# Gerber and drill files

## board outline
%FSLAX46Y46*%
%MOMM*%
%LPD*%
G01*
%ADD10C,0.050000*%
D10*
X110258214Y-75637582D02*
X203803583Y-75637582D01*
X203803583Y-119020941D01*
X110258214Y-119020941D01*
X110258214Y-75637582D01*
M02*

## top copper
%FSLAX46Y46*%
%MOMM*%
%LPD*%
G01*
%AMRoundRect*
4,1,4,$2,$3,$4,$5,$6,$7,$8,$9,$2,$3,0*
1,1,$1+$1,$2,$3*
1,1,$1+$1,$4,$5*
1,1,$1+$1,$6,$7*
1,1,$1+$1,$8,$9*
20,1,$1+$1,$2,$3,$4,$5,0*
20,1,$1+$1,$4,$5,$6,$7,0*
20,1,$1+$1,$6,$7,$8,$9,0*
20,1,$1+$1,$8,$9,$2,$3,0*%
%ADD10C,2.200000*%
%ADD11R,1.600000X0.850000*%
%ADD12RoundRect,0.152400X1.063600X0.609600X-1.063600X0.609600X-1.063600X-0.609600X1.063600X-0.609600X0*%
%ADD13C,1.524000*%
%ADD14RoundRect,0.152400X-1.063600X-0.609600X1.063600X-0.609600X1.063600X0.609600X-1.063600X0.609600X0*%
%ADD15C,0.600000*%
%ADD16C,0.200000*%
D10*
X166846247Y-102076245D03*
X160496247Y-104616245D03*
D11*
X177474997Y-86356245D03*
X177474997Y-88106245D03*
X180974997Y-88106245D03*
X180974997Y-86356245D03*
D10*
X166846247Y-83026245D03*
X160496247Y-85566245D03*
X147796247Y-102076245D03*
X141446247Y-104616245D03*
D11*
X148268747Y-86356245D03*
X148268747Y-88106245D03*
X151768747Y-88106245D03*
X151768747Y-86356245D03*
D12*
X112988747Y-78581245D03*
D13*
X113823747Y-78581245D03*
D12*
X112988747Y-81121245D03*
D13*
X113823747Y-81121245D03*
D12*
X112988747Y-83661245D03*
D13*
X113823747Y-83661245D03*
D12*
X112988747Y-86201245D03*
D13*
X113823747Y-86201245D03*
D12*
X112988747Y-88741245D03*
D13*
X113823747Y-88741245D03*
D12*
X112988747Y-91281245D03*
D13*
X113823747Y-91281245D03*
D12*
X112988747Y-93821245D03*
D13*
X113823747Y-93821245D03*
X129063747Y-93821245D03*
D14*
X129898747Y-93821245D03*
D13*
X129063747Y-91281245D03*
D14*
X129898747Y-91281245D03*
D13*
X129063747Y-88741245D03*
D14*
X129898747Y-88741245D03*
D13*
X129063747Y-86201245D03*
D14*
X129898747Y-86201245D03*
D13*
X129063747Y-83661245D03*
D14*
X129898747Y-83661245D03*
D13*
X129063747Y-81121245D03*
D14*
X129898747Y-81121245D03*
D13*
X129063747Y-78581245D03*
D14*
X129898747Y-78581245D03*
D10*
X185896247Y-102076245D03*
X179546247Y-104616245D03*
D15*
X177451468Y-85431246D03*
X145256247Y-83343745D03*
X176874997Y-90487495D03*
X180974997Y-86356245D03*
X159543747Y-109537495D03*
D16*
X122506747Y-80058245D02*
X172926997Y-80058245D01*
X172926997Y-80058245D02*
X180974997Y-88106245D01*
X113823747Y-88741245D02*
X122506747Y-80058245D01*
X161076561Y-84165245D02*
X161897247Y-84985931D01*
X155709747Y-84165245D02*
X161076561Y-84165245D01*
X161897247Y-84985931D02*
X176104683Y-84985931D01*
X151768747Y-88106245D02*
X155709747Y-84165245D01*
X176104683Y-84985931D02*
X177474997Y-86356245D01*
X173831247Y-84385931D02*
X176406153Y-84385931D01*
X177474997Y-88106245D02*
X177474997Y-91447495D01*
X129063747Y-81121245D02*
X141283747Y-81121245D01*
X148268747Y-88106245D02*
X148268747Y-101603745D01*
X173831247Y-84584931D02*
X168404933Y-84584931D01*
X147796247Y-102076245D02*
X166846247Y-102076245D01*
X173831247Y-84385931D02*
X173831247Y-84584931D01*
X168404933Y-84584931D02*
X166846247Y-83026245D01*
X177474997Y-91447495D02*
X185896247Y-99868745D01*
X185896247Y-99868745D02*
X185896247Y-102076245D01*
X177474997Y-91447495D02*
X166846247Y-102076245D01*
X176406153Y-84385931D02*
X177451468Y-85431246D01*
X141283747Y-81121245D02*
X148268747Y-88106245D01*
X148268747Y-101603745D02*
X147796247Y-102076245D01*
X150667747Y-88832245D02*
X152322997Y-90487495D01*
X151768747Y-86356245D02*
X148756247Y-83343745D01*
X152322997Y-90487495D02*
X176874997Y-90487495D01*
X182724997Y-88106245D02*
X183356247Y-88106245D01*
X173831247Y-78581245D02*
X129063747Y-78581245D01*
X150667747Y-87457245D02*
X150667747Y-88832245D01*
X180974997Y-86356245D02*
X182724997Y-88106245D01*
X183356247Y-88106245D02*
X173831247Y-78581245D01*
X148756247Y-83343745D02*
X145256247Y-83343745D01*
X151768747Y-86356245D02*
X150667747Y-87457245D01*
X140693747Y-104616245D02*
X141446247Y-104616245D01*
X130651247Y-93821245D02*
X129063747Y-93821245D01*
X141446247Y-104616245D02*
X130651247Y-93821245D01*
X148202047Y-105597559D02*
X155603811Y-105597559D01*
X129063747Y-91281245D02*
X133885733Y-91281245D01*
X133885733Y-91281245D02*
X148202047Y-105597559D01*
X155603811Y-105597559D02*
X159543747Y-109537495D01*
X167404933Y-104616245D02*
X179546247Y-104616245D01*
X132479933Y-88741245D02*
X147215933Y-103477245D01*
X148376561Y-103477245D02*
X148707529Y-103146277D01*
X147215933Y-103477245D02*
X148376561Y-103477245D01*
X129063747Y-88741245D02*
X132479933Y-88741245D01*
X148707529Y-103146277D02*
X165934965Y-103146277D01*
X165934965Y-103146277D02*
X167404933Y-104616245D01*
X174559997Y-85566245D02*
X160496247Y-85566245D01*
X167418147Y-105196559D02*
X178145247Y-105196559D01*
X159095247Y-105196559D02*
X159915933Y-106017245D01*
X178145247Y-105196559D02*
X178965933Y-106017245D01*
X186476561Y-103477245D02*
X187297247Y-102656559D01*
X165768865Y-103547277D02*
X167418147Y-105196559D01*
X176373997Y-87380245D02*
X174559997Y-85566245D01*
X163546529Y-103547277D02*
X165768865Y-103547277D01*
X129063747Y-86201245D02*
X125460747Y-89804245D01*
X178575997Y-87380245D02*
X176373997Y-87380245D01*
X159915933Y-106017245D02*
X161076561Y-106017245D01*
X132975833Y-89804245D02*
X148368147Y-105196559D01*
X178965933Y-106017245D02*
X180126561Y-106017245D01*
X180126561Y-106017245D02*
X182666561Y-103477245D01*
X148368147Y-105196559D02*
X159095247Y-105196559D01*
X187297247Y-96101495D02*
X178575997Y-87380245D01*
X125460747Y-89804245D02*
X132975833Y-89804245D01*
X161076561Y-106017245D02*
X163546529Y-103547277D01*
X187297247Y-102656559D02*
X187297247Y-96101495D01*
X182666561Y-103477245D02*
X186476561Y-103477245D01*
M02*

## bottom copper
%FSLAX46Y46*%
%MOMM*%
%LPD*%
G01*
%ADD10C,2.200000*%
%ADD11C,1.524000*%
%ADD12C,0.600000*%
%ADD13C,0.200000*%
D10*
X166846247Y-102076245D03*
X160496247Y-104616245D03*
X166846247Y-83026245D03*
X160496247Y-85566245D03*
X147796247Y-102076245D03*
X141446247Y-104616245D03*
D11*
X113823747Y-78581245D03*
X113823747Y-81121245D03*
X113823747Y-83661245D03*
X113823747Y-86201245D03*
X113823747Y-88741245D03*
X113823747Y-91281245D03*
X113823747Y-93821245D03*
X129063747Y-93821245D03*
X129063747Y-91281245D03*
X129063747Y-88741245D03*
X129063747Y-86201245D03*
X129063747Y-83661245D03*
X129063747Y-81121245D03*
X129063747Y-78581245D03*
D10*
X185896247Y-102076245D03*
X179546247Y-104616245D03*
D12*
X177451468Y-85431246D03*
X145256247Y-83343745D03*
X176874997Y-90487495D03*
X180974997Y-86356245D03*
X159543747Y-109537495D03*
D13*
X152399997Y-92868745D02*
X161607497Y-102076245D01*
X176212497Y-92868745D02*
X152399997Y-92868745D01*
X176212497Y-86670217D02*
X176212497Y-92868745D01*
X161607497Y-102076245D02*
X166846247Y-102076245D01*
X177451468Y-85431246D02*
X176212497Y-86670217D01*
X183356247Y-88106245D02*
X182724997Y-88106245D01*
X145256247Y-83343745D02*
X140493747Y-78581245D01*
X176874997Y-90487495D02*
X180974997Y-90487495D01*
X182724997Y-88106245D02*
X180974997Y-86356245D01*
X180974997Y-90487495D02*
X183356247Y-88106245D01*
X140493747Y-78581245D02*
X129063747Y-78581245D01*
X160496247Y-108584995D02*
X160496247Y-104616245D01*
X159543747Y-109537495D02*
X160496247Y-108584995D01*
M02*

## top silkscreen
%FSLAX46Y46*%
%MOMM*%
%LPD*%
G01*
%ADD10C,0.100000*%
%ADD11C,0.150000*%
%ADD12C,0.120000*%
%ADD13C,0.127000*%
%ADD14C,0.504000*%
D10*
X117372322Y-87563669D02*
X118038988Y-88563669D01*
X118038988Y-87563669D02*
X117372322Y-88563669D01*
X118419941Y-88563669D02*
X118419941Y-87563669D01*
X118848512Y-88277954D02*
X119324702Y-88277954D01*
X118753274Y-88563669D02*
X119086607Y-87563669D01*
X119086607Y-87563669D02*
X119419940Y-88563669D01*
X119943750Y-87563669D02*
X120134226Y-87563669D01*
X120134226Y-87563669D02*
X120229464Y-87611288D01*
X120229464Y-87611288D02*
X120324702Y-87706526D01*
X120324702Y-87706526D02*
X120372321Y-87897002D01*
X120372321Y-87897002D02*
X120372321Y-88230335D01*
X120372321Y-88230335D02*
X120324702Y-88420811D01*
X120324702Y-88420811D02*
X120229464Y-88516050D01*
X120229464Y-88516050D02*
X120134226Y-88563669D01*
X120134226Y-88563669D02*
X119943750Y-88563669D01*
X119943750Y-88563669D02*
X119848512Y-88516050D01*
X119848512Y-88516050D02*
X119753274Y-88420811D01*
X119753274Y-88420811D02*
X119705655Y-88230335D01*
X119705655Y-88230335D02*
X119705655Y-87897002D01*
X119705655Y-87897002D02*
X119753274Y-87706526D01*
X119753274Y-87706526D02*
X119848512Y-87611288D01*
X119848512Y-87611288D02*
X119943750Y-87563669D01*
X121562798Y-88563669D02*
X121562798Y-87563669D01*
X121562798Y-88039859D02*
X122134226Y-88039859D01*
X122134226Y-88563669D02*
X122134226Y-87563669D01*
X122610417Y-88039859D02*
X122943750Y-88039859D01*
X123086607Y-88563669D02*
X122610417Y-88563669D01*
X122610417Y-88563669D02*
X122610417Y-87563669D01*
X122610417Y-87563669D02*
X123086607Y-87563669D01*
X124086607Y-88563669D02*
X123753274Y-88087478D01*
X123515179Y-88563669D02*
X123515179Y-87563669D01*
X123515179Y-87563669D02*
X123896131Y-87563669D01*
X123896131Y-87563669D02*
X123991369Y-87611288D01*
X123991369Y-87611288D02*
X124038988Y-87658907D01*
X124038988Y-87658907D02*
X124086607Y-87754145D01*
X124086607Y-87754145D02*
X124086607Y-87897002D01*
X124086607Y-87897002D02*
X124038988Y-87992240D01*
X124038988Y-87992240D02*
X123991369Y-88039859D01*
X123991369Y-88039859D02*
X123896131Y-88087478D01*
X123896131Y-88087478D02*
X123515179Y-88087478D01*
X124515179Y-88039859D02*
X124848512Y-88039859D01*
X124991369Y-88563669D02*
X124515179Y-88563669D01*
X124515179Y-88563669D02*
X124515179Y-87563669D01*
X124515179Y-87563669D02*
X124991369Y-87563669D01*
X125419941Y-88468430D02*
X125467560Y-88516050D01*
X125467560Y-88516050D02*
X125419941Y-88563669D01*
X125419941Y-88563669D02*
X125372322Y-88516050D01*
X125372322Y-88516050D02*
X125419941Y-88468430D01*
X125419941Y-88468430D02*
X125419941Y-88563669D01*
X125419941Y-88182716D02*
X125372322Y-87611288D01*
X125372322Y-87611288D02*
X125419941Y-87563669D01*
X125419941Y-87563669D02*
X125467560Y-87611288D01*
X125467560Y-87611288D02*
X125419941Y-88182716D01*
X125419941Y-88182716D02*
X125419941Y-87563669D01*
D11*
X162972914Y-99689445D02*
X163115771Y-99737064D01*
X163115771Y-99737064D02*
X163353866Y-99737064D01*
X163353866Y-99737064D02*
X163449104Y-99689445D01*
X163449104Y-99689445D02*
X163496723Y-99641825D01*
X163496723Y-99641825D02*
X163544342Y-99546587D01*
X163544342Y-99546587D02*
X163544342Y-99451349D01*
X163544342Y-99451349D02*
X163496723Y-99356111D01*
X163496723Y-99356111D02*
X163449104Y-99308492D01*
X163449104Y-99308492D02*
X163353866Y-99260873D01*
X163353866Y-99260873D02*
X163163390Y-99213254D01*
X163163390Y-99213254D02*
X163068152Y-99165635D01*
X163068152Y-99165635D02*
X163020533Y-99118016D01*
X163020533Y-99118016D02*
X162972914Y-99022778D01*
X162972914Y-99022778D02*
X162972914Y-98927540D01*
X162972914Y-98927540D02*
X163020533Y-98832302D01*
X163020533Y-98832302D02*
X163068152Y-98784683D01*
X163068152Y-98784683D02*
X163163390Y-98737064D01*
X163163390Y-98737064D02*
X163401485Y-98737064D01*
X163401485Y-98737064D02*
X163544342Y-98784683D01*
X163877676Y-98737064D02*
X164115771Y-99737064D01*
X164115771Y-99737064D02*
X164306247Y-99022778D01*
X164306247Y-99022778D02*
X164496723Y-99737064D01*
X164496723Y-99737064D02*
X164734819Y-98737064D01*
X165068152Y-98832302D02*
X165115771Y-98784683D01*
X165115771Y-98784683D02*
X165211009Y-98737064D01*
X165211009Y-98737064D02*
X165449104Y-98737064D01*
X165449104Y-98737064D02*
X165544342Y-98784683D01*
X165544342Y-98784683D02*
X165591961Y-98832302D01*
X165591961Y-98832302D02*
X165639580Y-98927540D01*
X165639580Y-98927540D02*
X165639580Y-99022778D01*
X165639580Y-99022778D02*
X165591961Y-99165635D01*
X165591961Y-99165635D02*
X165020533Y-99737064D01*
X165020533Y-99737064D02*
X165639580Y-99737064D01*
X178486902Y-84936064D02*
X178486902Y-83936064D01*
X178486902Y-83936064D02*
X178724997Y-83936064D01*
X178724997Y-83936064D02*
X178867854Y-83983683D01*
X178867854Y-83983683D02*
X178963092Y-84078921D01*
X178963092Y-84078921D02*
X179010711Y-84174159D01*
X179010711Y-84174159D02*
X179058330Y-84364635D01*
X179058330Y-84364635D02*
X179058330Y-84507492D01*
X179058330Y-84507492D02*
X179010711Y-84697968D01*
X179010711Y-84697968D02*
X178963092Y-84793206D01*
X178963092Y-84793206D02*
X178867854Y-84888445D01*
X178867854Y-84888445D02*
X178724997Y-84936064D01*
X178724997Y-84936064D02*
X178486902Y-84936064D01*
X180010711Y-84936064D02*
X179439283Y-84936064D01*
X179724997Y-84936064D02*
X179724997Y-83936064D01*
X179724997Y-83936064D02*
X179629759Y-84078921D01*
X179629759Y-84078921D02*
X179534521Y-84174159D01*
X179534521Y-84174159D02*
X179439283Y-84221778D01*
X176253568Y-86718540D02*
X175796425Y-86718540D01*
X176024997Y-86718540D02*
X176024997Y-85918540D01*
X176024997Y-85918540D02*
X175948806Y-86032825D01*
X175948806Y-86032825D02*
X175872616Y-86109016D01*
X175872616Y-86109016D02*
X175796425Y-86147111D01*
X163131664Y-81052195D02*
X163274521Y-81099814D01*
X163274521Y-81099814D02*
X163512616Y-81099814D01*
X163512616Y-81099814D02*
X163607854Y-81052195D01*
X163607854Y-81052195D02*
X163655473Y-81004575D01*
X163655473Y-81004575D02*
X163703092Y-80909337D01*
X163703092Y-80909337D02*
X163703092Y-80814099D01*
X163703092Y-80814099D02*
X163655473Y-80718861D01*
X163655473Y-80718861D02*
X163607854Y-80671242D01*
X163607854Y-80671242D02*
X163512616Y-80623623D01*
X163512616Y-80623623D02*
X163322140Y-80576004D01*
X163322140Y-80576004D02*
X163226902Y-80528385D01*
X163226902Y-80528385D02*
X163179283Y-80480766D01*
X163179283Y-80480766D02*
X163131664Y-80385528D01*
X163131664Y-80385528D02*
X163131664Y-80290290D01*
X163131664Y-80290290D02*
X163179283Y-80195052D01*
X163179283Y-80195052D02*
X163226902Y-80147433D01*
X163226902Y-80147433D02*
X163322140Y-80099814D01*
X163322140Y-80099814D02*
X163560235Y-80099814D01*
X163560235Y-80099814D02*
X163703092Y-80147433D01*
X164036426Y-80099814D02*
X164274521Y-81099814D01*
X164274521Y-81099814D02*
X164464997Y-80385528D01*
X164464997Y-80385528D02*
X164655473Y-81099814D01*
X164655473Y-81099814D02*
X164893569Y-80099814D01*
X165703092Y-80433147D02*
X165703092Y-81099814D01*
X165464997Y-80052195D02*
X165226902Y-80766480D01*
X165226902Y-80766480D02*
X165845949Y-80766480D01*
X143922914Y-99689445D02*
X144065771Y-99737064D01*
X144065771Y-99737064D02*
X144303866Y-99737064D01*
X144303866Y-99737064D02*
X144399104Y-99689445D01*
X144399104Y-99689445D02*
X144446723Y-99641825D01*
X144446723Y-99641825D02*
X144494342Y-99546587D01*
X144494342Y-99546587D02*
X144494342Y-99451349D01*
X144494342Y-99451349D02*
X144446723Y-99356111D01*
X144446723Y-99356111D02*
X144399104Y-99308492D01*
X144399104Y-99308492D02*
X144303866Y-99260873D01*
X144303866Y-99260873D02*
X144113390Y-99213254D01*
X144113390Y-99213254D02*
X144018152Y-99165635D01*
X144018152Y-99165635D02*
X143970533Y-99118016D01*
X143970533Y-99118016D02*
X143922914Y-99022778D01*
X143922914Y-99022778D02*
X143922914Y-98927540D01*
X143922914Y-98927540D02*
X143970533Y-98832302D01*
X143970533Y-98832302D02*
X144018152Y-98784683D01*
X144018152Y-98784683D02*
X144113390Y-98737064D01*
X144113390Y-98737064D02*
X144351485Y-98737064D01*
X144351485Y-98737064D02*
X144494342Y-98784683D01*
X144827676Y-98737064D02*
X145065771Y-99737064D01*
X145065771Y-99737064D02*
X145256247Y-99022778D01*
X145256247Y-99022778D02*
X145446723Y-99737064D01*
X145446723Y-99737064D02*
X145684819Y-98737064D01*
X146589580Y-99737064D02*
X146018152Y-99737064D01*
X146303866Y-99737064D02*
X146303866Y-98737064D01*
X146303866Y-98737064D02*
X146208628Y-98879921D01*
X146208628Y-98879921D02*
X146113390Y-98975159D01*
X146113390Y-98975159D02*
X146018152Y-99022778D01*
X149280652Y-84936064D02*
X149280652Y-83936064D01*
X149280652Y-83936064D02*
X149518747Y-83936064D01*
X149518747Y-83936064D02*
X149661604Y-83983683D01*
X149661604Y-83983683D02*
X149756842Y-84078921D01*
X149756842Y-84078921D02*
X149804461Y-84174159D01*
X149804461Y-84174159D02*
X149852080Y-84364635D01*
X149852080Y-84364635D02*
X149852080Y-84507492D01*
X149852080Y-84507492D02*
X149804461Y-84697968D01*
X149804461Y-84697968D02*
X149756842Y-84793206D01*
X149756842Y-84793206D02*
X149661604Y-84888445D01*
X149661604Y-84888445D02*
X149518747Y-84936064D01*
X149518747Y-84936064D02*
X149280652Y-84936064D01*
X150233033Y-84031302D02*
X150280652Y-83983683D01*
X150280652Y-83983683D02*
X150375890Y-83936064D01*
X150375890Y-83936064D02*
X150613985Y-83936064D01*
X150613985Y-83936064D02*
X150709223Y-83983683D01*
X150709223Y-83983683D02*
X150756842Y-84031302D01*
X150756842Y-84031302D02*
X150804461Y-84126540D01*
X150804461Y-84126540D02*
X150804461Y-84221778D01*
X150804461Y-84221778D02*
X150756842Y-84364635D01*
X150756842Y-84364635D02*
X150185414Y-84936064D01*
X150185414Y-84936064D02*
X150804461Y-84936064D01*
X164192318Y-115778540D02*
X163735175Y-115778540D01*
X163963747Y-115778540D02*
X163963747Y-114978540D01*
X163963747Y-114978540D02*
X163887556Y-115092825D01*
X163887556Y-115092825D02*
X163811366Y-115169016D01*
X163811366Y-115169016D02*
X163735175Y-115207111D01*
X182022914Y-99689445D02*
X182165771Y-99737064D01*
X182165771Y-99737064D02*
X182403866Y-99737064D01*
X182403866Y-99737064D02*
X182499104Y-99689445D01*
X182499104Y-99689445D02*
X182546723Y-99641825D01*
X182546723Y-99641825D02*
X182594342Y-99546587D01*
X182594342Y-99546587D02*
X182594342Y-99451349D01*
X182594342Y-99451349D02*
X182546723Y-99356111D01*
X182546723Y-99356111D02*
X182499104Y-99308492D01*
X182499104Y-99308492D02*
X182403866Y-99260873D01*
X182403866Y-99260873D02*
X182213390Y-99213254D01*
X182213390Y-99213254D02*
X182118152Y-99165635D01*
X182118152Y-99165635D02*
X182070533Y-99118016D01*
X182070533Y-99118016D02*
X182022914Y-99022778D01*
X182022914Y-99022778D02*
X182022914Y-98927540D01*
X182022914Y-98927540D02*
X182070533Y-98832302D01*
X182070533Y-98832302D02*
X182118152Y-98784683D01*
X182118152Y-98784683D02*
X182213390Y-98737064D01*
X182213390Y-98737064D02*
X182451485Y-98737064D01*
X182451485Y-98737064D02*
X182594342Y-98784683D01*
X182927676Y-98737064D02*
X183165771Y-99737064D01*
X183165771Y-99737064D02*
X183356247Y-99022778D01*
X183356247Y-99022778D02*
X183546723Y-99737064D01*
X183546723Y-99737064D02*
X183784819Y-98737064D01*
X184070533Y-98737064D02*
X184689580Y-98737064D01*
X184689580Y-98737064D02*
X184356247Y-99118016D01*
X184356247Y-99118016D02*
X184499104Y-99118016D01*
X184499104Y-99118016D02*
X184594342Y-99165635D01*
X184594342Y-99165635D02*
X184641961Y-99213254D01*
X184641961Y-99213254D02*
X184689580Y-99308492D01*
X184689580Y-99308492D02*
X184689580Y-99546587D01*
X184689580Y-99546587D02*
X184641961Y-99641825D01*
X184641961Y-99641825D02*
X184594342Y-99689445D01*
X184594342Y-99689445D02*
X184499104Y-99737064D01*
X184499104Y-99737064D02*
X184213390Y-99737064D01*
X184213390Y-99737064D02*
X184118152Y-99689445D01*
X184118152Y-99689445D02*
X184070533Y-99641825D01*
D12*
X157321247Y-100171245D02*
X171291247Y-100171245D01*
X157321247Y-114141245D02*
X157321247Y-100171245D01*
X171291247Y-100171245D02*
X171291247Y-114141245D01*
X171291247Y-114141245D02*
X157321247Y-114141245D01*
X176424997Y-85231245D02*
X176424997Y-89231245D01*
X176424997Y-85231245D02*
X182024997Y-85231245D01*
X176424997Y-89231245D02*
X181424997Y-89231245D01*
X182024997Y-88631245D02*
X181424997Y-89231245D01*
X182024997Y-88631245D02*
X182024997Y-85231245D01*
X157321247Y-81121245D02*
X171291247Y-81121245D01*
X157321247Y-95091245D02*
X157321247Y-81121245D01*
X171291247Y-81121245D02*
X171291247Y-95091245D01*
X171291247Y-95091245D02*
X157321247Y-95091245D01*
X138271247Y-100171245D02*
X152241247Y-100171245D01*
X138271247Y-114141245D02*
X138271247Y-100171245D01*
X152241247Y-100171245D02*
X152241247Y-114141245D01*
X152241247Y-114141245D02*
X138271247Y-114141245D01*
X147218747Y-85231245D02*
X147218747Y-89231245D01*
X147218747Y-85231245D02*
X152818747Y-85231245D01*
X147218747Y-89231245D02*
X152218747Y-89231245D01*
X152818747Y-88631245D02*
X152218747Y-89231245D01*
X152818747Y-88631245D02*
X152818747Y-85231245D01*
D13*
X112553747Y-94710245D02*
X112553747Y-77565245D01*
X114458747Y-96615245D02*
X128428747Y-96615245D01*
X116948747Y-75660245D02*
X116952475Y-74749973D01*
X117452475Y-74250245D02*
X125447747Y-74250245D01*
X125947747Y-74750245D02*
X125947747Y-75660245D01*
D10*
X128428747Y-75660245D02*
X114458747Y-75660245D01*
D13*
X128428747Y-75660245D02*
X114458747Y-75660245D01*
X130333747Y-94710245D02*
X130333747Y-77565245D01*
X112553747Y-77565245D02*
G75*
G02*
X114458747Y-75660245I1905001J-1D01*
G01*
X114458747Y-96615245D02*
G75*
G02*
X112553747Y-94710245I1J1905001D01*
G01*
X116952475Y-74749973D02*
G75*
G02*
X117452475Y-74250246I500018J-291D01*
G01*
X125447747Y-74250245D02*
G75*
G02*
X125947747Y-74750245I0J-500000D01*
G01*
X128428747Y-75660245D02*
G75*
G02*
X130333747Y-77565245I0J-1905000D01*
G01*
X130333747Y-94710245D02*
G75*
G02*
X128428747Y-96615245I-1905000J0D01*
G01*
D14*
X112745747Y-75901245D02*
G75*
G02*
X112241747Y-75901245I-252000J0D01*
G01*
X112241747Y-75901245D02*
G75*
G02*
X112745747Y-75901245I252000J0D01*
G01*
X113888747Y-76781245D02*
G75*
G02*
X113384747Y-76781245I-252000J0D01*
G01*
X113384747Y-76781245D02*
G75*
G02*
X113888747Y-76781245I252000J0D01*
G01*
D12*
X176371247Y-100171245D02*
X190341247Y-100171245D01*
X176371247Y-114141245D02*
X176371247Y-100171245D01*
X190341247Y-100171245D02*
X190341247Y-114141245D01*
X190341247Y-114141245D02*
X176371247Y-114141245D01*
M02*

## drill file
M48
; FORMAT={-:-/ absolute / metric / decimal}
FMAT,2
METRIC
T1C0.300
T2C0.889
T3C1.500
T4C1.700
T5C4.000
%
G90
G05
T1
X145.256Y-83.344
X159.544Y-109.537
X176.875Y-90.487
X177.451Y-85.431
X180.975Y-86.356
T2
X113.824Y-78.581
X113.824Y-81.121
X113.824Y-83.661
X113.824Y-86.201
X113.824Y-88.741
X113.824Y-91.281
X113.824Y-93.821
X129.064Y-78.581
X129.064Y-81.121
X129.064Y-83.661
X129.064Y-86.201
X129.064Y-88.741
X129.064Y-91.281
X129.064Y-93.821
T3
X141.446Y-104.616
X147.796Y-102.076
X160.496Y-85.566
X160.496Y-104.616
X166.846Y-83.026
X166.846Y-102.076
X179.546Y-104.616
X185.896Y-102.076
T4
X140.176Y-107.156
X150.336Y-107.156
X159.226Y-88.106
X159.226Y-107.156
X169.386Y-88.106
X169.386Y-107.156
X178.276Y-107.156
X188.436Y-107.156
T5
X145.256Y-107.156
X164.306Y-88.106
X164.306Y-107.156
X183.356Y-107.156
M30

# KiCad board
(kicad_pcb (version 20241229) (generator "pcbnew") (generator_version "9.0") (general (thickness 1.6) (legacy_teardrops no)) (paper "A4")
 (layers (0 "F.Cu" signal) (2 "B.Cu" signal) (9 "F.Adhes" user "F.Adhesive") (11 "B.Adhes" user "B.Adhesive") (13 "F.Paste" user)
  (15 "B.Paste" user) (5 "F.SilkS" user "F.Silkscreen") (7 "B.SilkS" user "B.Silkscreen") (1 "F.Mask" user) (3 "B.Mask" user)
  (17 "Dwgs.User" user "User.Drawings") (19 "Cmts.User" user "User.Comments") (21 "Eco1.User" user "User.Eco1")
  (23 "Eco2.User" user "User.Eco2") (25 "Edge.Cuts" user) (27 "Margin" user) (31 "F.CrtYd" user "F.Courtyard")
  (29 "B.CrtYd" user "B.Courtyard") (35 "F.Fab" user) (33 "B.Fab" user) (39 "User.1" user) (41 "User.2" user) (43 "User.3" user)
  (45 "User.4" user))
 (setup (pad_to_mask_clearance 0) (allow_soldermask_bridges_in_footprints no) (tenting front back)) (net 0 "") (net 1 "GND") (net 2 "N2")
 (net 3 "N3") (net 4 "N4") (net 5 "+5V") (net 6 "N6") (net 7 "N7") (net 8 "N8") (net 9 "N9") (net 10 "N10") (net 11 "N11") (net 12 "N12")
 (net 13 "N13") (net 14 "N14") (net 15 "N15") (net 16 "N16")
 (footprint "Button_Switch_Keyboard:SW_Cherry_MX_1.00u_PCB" (layer "F.Cu") (at 166.846247 102.076245)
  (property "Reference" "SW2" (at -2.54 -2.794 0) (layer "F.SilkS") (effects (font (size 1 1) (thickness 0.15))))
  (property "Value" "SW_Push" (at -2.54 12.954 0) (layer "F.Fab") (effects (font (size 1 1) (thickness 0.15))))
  (fp_line (start -9.525 -1.905) (end 4.445 -1.905) (stroke (width 0.12) (type solid)) (layer "F.SilkS"))
  (fp_line (start -9.525 12.065) (end -9.525 -1.905) (stroke (width 0.12) (type solid)) (layer "F.SilkS"))
  (fp_line (start 4.445 -1.905) (end 4.445 12.065) (stroke (width 0.12) (type solid)) (layer "F.SilkS"))
  (fp_line (start 4.445 12.065) (end -9.525 12.065) (stroke (width 0.12) (type solid)) (layer "F.SilkS"))
  (pad "" np_thru_hole circle (at -7.62 5.08) (size 1.7 1.7) (drill 1.7) (layers "*.Cu" "*.Mask"))
  (pad "" np_thru_hole circle (at -2.54 5.08) (size 4 4) (drill 4) (layers "*.Cu" "*.Mask"))
  (pad "" np_thru_hole circle (at 2.54 5.08) (size 1.7 1.7) (drill 1.7) (layers "*.Cu" "*.Mask"))
  (pad "1" thru_hole circle (at 0 0) (size 2.2 2.2) (drill 1.5) (layers "*.Cu" "*.Mask") (remove_unused_layers no) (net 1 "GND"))
  (pad "2" thru_hole circle (at -6.35 2.54) (size 2.2 2.2) (drill 1.5) (layers "*.Cu" "*.Mask") (remove_unused_layers no) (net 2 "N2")))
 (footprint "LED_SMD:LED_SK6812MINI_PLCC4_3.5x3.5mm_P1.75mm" (layer "F.Cu") (at 179.224997 87.231245)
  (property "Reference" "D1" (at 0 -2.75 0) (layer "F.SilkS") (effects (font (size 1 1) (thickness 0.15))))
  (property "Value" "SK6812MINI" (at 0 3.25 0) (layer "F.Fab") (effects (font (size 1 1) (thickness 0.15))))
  (fp_line (start -2.8 -2) (end -2.8 2) (stroke (width 0.12) (type default)) (layer "F.SilkS"))
  (fp_line (start -2.8 -2) (end 2.8 -2) (stroke (width 0.12) (type solid)) (layer "F.SilkS"))
  (fp_line (start -2.8 2) (end 2.2 2) (stroke (width 0.12) (type solid)) (layer "F.SilkS"))
  (fp_line (start 2.8 1.4) (end 2.2 2) (stroke (width 0.12) (type default)) (layer "F.SilkS"))
  (fp_line (start 2.8 1.4) (end 2.8 -2) (stroke (width 0.12) (type solid)) (layer "F.SilkS"))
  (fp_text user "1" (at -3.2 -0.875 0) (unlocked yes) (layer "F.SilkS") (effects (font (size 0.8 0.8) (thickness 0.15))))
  (pad "1" smd rect (at -1.75 -0.875) (size 1.6 0.85) (layers "F.Cu" "F.Mask" "F.Paste") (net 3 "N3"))
  (pad "2" smd rect (at -1.75 0.875) (size 1.6 0.85) (layers "F.Cu" "F.Mask" "F.Paste") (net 1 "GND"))
  (pad "3" smd rect (at 1.75 0.875) (size 1.6 0.85) (layers "F.Cu" "F.Mask" "F.Paste") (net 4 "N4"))
  (pad "4" smd rect (at 1.75 -0.875) (size 1.6 0.85) (layers "F.Cu" "F.Mask" "F.Paste") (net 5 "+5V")))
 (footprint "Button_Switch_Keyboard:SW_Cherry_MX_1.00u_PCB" (layer "F.Cu") (at 166.846247 83.026245)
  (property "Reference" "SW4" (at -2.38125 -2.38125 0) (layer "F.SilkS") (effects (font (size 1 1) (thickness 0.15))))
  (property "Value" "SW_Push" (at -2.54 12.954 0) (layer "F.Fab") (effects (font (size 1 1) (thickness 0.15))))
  (fp_line (start -9.525 -1.905) (end 4.445 -1.905) (stroke (width 0.12) (type solid)) (layer "F.SilkS"))
  (fp_line (start -9.525 12.065) (end -9.525 -1.905) (stroke (width 0.12) (type solid)) (layer "F.SilkS"))
  (fp_line (start 4.445 -1.905) (end 4.445 12.065) (stroke (width 0.12) (type solid)) (layer "F.SilkS"))
  (fp_line (start 4.445 12.065) (end -9.525 12.065) (stroke (width 0.12) (type solid)) (layer "F.SilkS"))
  (pad "" np_thru_hole circle (at -7.62 5.08) (size 1.7 1.7) (drill 1.7) (layers "*.Cu" "*.Mask"))
  (pad "" np_thru_hole circle (at -2.54 5.08) (size 4 4) (drill 4) (layers "*.Cu" "*.Mask"))
  (pad "" np_thru_hole circle (at 2.54 5.08) (size 1.7 1.7) (drill 1.7) (layers "*.Cu" "*.Mask"))
  (pad "1" thru_hole circle (at 0 0) (size 2.2 2.2) (drill 1.5) (layers "*.Cu" "*.Mask") (remove_unused_layers no) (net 1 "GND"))
  (pad "2" thru_hole circle (at -6.35 2.54) (size 2.2 2.2) (drill 1.5) (layers "*.Cu" "*.Mask") (remove_unused_layers no) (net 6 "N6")))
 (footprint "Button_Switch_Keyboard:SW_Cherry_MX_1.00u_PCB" (layer "F.Cu") (at 147.796247 102.076245)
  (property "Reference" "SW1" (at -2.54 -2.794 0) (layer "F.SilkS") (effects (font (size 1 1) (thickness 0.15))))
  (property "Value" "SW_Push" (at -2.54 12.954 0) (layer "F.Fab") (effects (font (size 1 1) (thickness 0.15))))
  (fp_line (start -9.525 -1.905) (end 4.445 -1.905) (stroke (width 0.12) (type solid)) (layer "F.SilkS"))
  (fp_line (start -9.525 12.065) (end -9.525 -1.905) (stroke (width 0.12) (type solid)) (layer "F.SilkS"))
  (fp_line (start 4.445 -1.905) (end 4.445 12.065) (stroke (width 0.12) (type solid)) (layer "F.SilkS"))
  (fp_line (start 4.445 12.065) (end -9.525 12.065) (stroke (width 0.12) (type solid)) (layer "F.SilkS"))
  (pad "" np_thru_hole circle (at -7.62 5.08) (size 1.7 1.7) (drill 1.7) (layers "*.Cu" "*.Mask"))
  (pad "" np_thru_hole circle (at -2.54 5.08) (size 4 4) (drill 4) (layers "*.Cu" "*.Mask"))
  (pad "" np_thru_hole circle (at 2.54 5.08) (size 1.7 1.7) (drill 1.7) (layers "*.Cu" "*.Mask"))
  (pad "1" thru_hole circle (at 0 0) (size 2.2 2.2) (drill 1.5) (layers "*.Cu" "*.Mask") (remove_unused_layers no) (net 1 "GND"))
  (pad "2" thru_hole circle (at -6.35 2.54) (size 2.2 2.2) (drill 1.5) (layers "*.Cu" "*.Mask") (remove_unused_layers no) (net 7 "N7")))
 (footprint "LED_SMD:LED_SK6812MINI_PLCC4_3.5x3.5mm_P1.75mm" (layer "F.Cu") (at 150.018747 87.231245)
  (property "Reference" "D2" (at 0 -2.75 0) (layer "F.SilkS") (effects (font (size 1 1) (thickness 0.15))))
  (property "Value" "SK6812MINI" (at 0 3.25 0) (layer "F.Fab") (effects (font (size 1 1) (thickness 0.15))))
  (fp_line (start -2.8 -2) (end -2.8 2) (stroke (width 0.12) (type default)) (layer "F.SilkS"))
  (fp_line (start -2.8 -2) (end 2.8 -2) (stroke (width 0.12) (type solid)) (layer "F.SilkS"))
  (fp_line (start -2.8 2) (end 2.2 2) (stroke (width 0.12) (type solid)) (layer "F.SilkS"))
  (fp_line (start 2.8 1.4) (end 2.2 2) (stroke (width 0.12) (type default)) (layer "F.SilkS"))
  (fp_line (start 2.8 1.4) (end 2.8 -2) (stroke (width 0.12) (type solid)) (layer "F.SilkS"))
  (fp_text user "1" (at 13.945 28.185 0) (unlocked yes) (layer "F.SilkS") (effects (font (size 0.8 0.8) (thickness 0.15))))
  (pad "1" smd rect (at -1.75 -0.875) (size 1.6 0.85) (layers "F.Cu" "F.Mask" "F.Paste") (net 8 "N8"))
  (pad "2" smd rect (at -1.75 0.875) (size 1.6 0.85) (layers "F.Cu" "F.Mask" "F.Paste") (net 1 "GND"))
  (pad "3" smd rect (at 1.75 0.875) (size 1.6 0.85) (layers "F.Cu" "F.Mask" "F.Paste") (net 3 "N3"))
  (pad "4" smd rect (at 1.75 -0.875) (size 1.6 0.85) (layers "F.Cu" "F.Mask" "F.Paste") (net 5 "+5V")))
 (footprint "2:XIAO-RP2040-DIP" (layer "F.Cu") (at 121.443747 86.201245)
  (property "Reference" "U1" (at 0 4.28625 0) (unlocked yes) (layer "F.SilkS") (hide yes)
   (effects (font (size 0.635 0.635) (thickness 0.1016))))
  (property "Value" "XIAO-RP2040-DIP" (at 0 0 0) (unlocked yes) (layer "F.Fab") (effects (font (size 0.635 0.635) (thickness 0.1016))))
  (fp_line (start -8.89 8.509) (end -8.89 -8.636) (stroke (width 0.127) (type solid)) (layer "F.SilkS"))
  (fp_line (start -6.985 10.414) (end 6.985 10.414) (stroke (width 0.127) (type solid)) (layer "F.SilkS"))
  (fp_line (start -4.495 -10.541) (end -4.491272 -11.451272) (stroke (width 0.127) (type solid)) (layer "F.SilkS"))
  (fp_line (start -3.991272 -11.951) (end 4.004 -11.951) (stroke (width 0.127) (type solid)) (layer "F.SilkS"))
  (fp_line (start 4.504 -11.451) (end 4.504 -10.541) (stroke (width 0.127) (type solid)) (layer "F.SilkS"))
  (fp_line (start 6.985 -10.541) (end -6.985 -10.541) (stroke (width 0.1) (type solid)) (layer "F.SilkS"))
  (fp_line (start 6.985 -10.541) (end -6.985 -10.541) (stroke (width 0.127) (type solid)) (layer "F.SilkS"))
  (fp_line (start 8.89 8.509) (end 8.89 -8.636) (stroke (width 0.127) (type solid)) (layer "F.SilkS"))
  (fp_arc (start -8.89 -8.636) (mid -8.332038 -9.983038) (end -6.985 -10.541) (stroke (width 0.127) (type solid)) (layer "F.SilkS"))
  (fp_arc (start -6.985 10.414) (mid -8.332038 9.856038) (end -8.89 8.509) (stroke (width 0.127) (type solid)) (layer "F.SilkS"))
  (fp_arc (start -4.491272 -11.451272) (mid -4.344728 -11.80464) (end -3.991272 -11.951) (stroke (width 0.127) (type default))
   (layer "F.SilkS"))
  (fp_arc (start 4.004 -11.951) (mid 4.357553 -11.804553) (end 4.504 -11.451) (stroke (width 0.127) (type default)) (layer "F.SilkS"))
  (fp_arc (start 6.985 -10.541) (mid 8.332038 -9.983038) (end 8.89 -8.636) (stroke (width 0.127) (type solid)) (layer "F.SilkS"))
  (fp_arc (start 8.89 8.509) (mid 8.332038 9.856038) (end 6.985 10.414) (stroke (width 0.127) (type solid)) (layer "F.SilkS"))
  (fp_circle (center -8.95 -10.3) (end -8.95 -10.554) (stroke (width 0.5) (type solid)) (fill yes) (layer "F.SilkS"))
  (fp_circle (center -7.807 -9.42) (end -7.807 -9.674) (stroke (width 0.5) (type solid)) (fill yes) (layer "F.SilkS"))
  (pad "1" smd roundrect (at -8.455 -7.62 180) (size 2.432 1.524) (layers "F.Cu" "F.Mask") (roundrect_rratio 0.1) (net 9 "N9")
   (thermal_bridge_angle 45))
  (pad "1" thru_hole circle (at -7.62 -7.62 180) (size 1.524 1.524) (drill 0.889) (layers "*.Cu" "*.Mask") (remove_unused_layers no)
   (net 9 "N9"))
  (pad "2" smd roundrect (at -8.455 -5.08 180) (size 2.432 1.524) (layers "F.Cu" "F.Mask") (roundrect_rratio 0.1) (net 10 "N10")
   (thermal_bridge_angle 45))
  (pad "2" thru_hole circle (at -7.62 -5.08 180) (size 1.524 1.524) (drill 0.889) (layers "*.Cu" "*.Mask") (remove_unused_layers no)
   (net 10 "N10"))
  (pad "3" smd roundrect (at -8.455 -2.54 180) (size 2.432 1.524) (layers "F.Cu" "F.Mask") (roundrect_rratio 0.1) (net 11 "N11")
   (thermal_bridge_angle 45))
  (pad "3" thru_hole circle (at -7.62 -2.54 180) (size 1.524 1.524) (drill 0.889) (layers "*.Cu" "*.Mask") (remove_unused_layers no)
   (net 11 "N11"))
  (pad "4" smd roundrect (at -8.455 0 180) (size 2.432 1.524) (layers "F.Cu" "F.Mask") (roundrect_rratio 0.1) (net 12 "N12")
   (thermal_bridge_angle 45))
  (pad "4" thru_hole circle (at -7.62 0 180) (size 1.524 1.524) (drill 0.889) (layers "*.Cu" "*.Mask") (remove_unused_layers no)
   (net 12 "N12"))
  (pad "5" smd roundrect (at -8.455 2.54 180) (size 2.432 1.524) (layers "F.Cu" "F.Mask") (roundrect_rratio 0.1) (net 4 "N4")
   (thermal_bridge_angle 45))
  (pad "5" thru_hole circle (at -7.62 2.54 180) (size 1.524 1.524) (drill 0.889) (layers "*.Cu" "*.Mask") (remove_unused_layers no)
   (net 4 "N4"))
  (pad "6" smd roundrect (at -8.455 5.08 180) (size 2.432 1.524) (layers "F.Cu" "F.Mask") (roundrect_rratio 0.1) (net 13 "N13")
   (thermal_bridge_angle 45))
  (pad "6" thru_hole circle (at -7.62 5.08 180) (size 1.524 1.524) (drill 0.889) (layers "*.Cu" "*.Mask") (remove_unused_layers no)
   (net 13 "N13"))
  (pad "7" smd roundrect (at -8.455 7.62 180) (size 2.432 1.524) (layers "F.Cu" "F.Mask") (roundrect_rratio 0.1) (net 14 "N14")
   (thermal_bridge_angle 45))
  (pad "7" thru_hole circle (at -7.62 7.62 180) (size 1.524 1.524) (drill 0.889) (layers "*.Cu" "*.Mask") (remove_unused_layers no)
   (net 14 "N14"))
  (pad "8" thru_hole circle (at 7.62 7.62) (size 1.524 1.524) (drill 0.889) (layers "*.Cu" "*.Mask") (remove_unused_layers no) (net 7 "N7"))
  (pad "8" smd roundrect (at 8.455 7.62) (size 2.432 1.524) (layers "F.Cu" "F.Mask") (roundrect_rratio 0.1) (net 7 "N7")
   (thermal_bridge_angle 45))
  (pad "9" thru_hole circle (at 7.62 5.08) (size 1.524 1.524) (drill 0.889) (layers "*.Cu" "*.Mask") (remove_unused_layers no) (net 2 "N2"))
  (pad "9" smd roundrect (at 8.455 5.08) (size 2.432 1.524) (layers "F.Cu" "F.Mask") (roundrect_rratio 0.1) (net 2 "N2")
   (thermal_bridge_angle 45))
  (pad "10" thru_hole circle (at 7.62 2.54) (size 1.524 1.524) (drill 0.889) (layers "*.Cu" "*.Mask") (remove_unused_layers no)
   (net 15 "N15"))
  (pad "10" smd roundrect (at 8.455 2.54) (size 2.432 1.524) (layers "F.Cu" "F.Mask") (roundrect_rratio 0.1) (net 15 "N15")
   (thermal_bridge_angle 45))
  (pad "11" thru_hole circle (at 7.62 0) (size 1.524 1.524) (drill 0.889) (layers "*.Cu" "*.Mask") (remove_unused_layers no) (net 6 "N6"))
  (pad "11" smd roundrect (at 8.455 0) (size 2.432 1.524) (layers "F.Cu" "F.Mask") (roundrect_rratio 0.1) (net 6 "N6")
   (thermal_bridge_angle 45))
  (pad "12" thru_hole circle (at 7.62 -2.54) (size 1.524 1.524) (drill 0.889) (layers "*.Cu" "*.Mask") (remove_unused_layers no)
   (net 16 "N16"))
  (pad "12" smd roundrect (at 8.455 -2.54) (size 2.432 1.524) (layers "F.Cu" "F.Mask") (roundrect_rratio 0.1) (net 16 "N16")
   (thermal_bridge_angle 45))
  (pad "13" thru_hole circle (at 7.62 -5.08) (size 1.524 1.524) (drill 0.889) (layers "*.Cu" "*.Mask") (remove_unused_layers no)
   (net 1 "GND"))
  (pad "13" smd roundrect (at 8.455 -5.08) (size 2.432 1.524) (layers "F.Cu" "F.Mask") (roundrect_rratio 0.1) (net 1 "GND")
   (thermal_bridge_angle 45))
  (pad "14" thru_hole circle (at 7.62 -7.62) (size 1.524 1.524) (drill 0.889) (layers "*.Cu" "*.Mask") (remove_unused_layers no)
   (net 5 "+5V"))
  (pad "14" smd roundrect (at 8.455 -7.62) (size 2.432 1.524) (layers "F.Cu" "F.Mask") (roundrect_rratio 0.1) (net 5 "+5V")
   (thermal_bridge_angle 45)))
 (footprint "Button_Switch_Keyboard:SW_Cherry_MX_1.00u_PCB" (layer "F.Cu") (at 185.896247 102.076245)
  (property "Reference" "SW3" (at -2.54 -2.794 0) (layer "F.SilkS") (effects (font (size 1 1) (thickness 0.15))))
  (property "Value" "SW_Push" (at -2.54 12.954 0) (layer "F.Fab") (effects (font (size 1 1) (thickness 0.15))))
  (fp_line (start -9.525 -1.905) (end 4.445 -1.905) (stroke (width 0.12) (type solid)) (layer "F.SilkS"))
  (fp_line (start -9.525 12.065) (end -9.525 -1.905) (stroke (width 0.12) (type solid)) (layer "F.SilkS"))
  (fp_line (start 4.445 -1.905) (end 4.445 12.065) (stroke (width 0.12) (type solid)) (layer "F.SilkS"))
  (fp_line (start 4.445 12.065) (end -9.525 12.065) (stroke (width 0.12) (type solid)) (layer "F.SilkS"))
  (pad "" np_thru_hole circle (at -7.62 5.08) (size 1.7 1.7) (drill 1.7) (layers "*.Cu" "*.Mask"))
  (pad "" np_thru_hole circle (at -2.54 5.08) (size 4 4) (drill 4) (layers "*.Cu" "*.Mask"))
  (pad "" np_thru_hole circle (at 2.54 5.08) (size 1.7 1.7) (drill 1.7) (layers "*.Cu" "*.Mask"))
  (pad "1" thru_hole circle (at 0 0) (size 2.2 2.2) (drill 1.5) (layers "*.Cu" "*.Mask") (remove_unused_layers no) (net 1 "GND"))
  (pad "2" thru_hole circle (at -6.35 2.54) (size 2.2 2.2) (drill 1.5) (layers "*.Cu" "*.Mask") (remove_unused_layers no) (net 15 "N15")))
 (gr_rect (start 110.258214 75.637582) (end 203.803583 119.020941) (stroke (width 0.05) (type default)) (fill no) (layer "Edge.Cuts"))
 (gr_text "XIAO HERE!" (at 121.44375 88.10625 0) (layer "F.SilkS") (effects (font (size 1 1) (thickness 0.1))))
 (segment (start 122.506747 80.058245) (end 172.926997 80.058245) (width 0.2) (layer "F.Cu") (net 4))
 (segment (start 172.926997 80.058245) (end 180.974997 88.106245) (width 0.2) (layer "F.Cu") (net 4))
 (segment (start 113.823747 88.741245) (end 122.506747 80.058245) (width 0.2) (layer "F.Cu") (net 4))
 (segment (start 161.076561 84.165245) (end 161.897247 84.985931) (width 0.2) (layer "F.Cu") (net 3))
 (segment (start 155.709747 84.165245) (end 161.076561 84.165245) (width 0.2) (layer "F.Cu") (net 3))
 (segment (start 161.897247 84.985931) (end 176.104683 84.985931) (width 0.2) (layer "F.Cu") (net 3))
 (segment (start 151.768747 88.106245) (end 155.709747 84.165245) (width 0.2) (layer "F.Cu") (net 3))
 (segment (start 176.104683 84.985931) (end 177.474997 86.356245) (width 0.2) (layer "F.Cu") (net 3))
 (segment (start 173.831247 84.385931) (end 176.406153 84.385931) (width 0.2) (layer "F.Cu") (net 1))
 (segment (start 177.474997 88.106245) (end 177.474997 91.447495) (width 0.2) (layer "F.Cu") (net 1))
 (segment (start 129.063747 81.121245) (end 141.283747 81.121245) (width 0.2) (layer "F.Cu") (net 1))
 (segment (start 148.268747 88.106245) (end 148.268747 101.603745) (width 0.2) (layer "F.Cu") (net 1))
 (segment (start 173.831247 84.584931) (end 168.404933 84.584931) (width 0.2) (layer "F.Cu") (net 1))
 (segment (start 147.796247 102.076245) (end 166.846247 102.076245) (width 0.2) (layer "F.Cu") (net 1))
 (segment (start 173.831247 84.385931) (end 173.831247 84.584931) (width 0.2) (layer "F.Cu") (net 1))
 (segment (start 168.404933 84.584931) (end 166.846247 83.026245) (width 0.2) (layer "F.Cu") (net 1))
 (segment (start 177.474997 91.447495) (end 185.896247 99.868745) (width 0.2) (layer "F.Cu") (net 1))
 (segment (start 185.896247 99.868745) (end 185.896247 102.076245) (width 0.2) (layer "F.Cu") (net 1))
 (segment (start 177.474997 91.447495) (end 166.846247 102.076245) (width 0.2) (layer "F.Cu") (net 1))
 (segment (start 176.406153 84.385931) (end 177.451468 85.431246) (width 0.2) (layer "F.Cu") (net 1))
 (segment (start 141.283747 81.121245) (end 148.268747 88.106245) (width 0.2) (layer "F.Cu") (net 1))
 (segment (start 148.268747 101.603745) (end 147.796247 102.076245) (width 0.2) (layer "F.Cu") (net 1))
 (via (at 177.451468 85.431246) (size 0.6) (drill 0.3) (layers "F.Cu" "B.Cu") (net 1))
 (segment (start 152.399997 92.868745) (end 161.607497 102.076245) (width 0.2) (layer "B.Cu") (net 1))
 (segment (start 176.212497 92.868745) (end 152.399997 92.868745) (width 0.2) (layer "B.Cu") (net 1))
 (segment (start 176.212497 86.670217) (end 176.212497 92.868745) (width 0.2) (layer "B.Cu") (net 1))
 (segment (start 161.607497 102.076245) (end 166.846247 102.076245) (width 0.2) (layer "B.Cu") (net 1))
 (segment (start 177.451468 85.431246) (end 176.212497 86.670217) (width 0.2) (layer "B.Cu") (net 1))
 (segment (start 150.667747 88.832245) (end 152.322997 90.487495) (width 0.2) (layer "F.Cu") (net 5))
 (segment (start 151.768747 86.356245) (end 148.756247 83.343745) (width 0.2) (layer "F.Cu") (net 5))
 (segment (start 152.322997 90.487495) (end 176.874997 90.487495) (width 0.2) (layer "F.Cu") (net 5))
 (segment (start 182.724997 88.106245) (end 183.356247 88.106245) (width 0.2) (layer "F.Cu") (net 5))
 (segment (start 173.831247 78.581245) (end 129.063747 78.581245) (width 0.2) (layer "F.Cu") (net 5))
 (segment (start 150.667747 87.457245) (end 150.667747 88.832245) (width 0.2) (layer "F.Cu") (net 5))
 (segment (start 180.974997 86.356245) (end 182.724997 88.106245) (width 0.2) (layer "F.Cu") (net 5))
 (segment (start 183.356247 88.106245) (end 173.831247 78.581245) (width 0.2) (layer "F.Cu") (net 5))
 (segment (start 148.756247 83.343745) (end 145.256247 83.343745) (width 0.2) (layer "F.Cu") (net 5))
 (segment (start 151.768747 86.356245) (end 150.667747 87.457245) (width 0.2) (layer "F.Cu") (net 5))
 (via (at 145.256247 83.343745) (size 0.6) (drill 0.3) (layers "F.Cu" "B.Cu") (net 5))
 (via (at 176.874997 90.487495) (size 0.6) (drill 0.3) (layers "F.Cu" "B.Cu") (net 5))
 (via (at 180.974997 86.356245) (size 0.6) (drill 0.3) (layers "F.Cu" "B.Cu") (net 5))
 (segment (start 183.356247 88.106245) (end 182.724997 88.106245) (width 0.2) (layer "B.Cu") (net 5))
 (segment (start 145.256247 83.343745) (end 140.493747 78.581245) (width 0.2) (layer "B.Cu") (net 5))
 (segment (start 176.874997 90.487495) (end 180.974997 90.487495) (width 0.2) (layer "B.Cu") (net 5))
 (segment (start 182.724997 88.106245) (end 180.974997 86.356245) (width 0.2) (layer "B.Cu") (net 5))
 (segment (start 180.974997 90.487495) (end 183.356247 88.106245) (width 0.2) (layer "B.Cu") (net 5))
 (segment (start 140.493747 78.581245) (end 129.063747 78.581245) (width 0.2) (layer "B.Cu") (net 5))
 (segment (start 140.693747 104.616245) (end 141.446247 104.616245) (width 0.2) (layer "F.Cu") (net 7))
 (segment (start 130.651247 93.821245) (end 129.063747 93.821245) (width 0.2) (layer "F.Cu") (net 7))
 (segment (start 141.446247 104.616245) (end 130.651247 93.821245) (width 0.2) (layer "F.Cu") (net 7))
 (segment (start 148.202047 105.597559) (end 155.603811 105.597559) (width 0.2) (layer "F.Cu") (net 2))
 (segment (start 129.063747 91.281245) (end 133.885733 91.281245) (width 0.2) (layer "F.Cu") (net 2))
 (segment (start 133.885733 91.281245) (end 148.202047 105.597559) (width 0.2) (layer "F.Cu") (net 2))
 (segment (start 155.603811 105.597559) (end 159.543747 109.537495) (width 0.2) (layer "F.Cu") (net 2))
 (via (at 159.543747 109.537495) (size 0.6) (drill 0.3) (layers "F.Cu" "B.Cu") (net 2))
 (segment (start 160.496247 108.584995) (end 160.496247 104.616245) (width 0.2) (layer "B.Cu") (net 2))
 (segment (start 159.543747 109.537495) (end 160.496247 108.584995) (width 0.2) (layer "B.Cu") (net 2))
 (segment (start 167.404933 104.616245) (end 179.546247 104.616245) (width 0.2) (layer "F.Cu") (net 15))
 (segment (start 132.479933 88.741245) (end 147.215933 103.477245) (width 0.2) (layer "F.Cu") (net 15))
 (segment (start 148.376561 103.477245) (end 148.707529 103.146277) (width 0.2) (layer "F.Cu") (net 15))
 (segment (start 147.215933 103.477245) (end 148.376561 103.477245) (width 0.2) (layer "F.Cu") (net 15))
 (segment (start 129.063747 88.741245) (end 132.479933 88.741245) (width 0.2) (layer "F.Cu") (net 15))
 (segment (start 148.707529 103.146277) (end 165.934965 103.146277) (width 0.2) (layer "F.Cu") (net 15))
 (segment (start 165.934965 103.146277) (end 167.404933 104.616245) (width 0.2) (layer "F.Cu") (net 15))
 (segment (start 174.559997 85.566245) (end 160.496247 85.566245) (width 0.2) (layer "F.Cu") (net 6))
 (segment (start 167.418147 105.196559) (end 178.145247 105.196559) (width 0.2) (layer "F.Cu") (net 6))
 (segment (start 159.095247 105.196559) (end 159.915933 106.017245) (width 0.2) (layer "F.Cu") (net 6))
 (segment (start 178.145247 105.196559) (end 178.965933 106.017245) (width 0.2) (layer "F.Cu") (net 6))
 (segment (start 186.476561 103.477245) (end 187.297247 102.656559) (width 0.2) (layer "F.Cu") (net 6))
 (segment (start 165.768865 103.547277) (end 167.418147 105.196559) (width 0.2) (layer "F.Cu") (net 6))
 (segment (start 176.373997 87.380245) (end 174.559997 85.566245) (width 0.2) (layer "F.Cu") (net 6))
 (segment (start 163.546529 103.547277) (end 165.768865 103.547277) (width 0.2) (layer "F.Cu") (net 6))
 (segment (start 129.063747 86.201245) (end 125.460747 89.804245) (width 0.2) (layer "F.Cu") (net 6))
 (segment (start 178.575997 87.380245) (end 176.373997 87.380245) (width 0.2) (layer "F.Cu") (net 6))
 (segment (start 159.915933 106.017245) (end 161.076561 106.017245) (width 0.2) (layer "F.Cu") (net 6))
 (segment (start 132.975833 89.804245) (end 148.368147 105.196559) (width 0.2) (layer "F.Cu") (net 6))
 (segment (start 178.965933 106.017245) (end 180.126561 106.017245) (width 0.2) (layer "F.Cu") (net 6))
 (segment (start 180.126561 106.017245) (end 182.666561 103.477245) (width 0.2) (layer "F.Cu") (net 6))
 (segment (start 148.368147 105.196559) (end 159.095247 105.196559) (width 0.2) (layer "F.Cu") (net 6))
 (segment (start 187.297247 96.101495) (end 178.575997 87.380245) (width 0.2) (layer "F.Cu") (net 6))
 (segment (start 125.460747 89.804245) (end 132.975833 89.804245) (width 0.2) (layer "F.Cu") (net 6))
 (segment (start 161.076561 106.017245) (end 163.546529 103.547277) (width 0.2) (layer "F.Cu") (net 6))
 (segment (start 187.297247 102.656559) (end 187.297247 96.101495) (width 0.2) (layer "F.Cu") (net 6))
 (segment (start 182.666561 103.477245) (end 186.476561 103.477245) (width 0.2) (layer "F.Cu") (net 6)))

